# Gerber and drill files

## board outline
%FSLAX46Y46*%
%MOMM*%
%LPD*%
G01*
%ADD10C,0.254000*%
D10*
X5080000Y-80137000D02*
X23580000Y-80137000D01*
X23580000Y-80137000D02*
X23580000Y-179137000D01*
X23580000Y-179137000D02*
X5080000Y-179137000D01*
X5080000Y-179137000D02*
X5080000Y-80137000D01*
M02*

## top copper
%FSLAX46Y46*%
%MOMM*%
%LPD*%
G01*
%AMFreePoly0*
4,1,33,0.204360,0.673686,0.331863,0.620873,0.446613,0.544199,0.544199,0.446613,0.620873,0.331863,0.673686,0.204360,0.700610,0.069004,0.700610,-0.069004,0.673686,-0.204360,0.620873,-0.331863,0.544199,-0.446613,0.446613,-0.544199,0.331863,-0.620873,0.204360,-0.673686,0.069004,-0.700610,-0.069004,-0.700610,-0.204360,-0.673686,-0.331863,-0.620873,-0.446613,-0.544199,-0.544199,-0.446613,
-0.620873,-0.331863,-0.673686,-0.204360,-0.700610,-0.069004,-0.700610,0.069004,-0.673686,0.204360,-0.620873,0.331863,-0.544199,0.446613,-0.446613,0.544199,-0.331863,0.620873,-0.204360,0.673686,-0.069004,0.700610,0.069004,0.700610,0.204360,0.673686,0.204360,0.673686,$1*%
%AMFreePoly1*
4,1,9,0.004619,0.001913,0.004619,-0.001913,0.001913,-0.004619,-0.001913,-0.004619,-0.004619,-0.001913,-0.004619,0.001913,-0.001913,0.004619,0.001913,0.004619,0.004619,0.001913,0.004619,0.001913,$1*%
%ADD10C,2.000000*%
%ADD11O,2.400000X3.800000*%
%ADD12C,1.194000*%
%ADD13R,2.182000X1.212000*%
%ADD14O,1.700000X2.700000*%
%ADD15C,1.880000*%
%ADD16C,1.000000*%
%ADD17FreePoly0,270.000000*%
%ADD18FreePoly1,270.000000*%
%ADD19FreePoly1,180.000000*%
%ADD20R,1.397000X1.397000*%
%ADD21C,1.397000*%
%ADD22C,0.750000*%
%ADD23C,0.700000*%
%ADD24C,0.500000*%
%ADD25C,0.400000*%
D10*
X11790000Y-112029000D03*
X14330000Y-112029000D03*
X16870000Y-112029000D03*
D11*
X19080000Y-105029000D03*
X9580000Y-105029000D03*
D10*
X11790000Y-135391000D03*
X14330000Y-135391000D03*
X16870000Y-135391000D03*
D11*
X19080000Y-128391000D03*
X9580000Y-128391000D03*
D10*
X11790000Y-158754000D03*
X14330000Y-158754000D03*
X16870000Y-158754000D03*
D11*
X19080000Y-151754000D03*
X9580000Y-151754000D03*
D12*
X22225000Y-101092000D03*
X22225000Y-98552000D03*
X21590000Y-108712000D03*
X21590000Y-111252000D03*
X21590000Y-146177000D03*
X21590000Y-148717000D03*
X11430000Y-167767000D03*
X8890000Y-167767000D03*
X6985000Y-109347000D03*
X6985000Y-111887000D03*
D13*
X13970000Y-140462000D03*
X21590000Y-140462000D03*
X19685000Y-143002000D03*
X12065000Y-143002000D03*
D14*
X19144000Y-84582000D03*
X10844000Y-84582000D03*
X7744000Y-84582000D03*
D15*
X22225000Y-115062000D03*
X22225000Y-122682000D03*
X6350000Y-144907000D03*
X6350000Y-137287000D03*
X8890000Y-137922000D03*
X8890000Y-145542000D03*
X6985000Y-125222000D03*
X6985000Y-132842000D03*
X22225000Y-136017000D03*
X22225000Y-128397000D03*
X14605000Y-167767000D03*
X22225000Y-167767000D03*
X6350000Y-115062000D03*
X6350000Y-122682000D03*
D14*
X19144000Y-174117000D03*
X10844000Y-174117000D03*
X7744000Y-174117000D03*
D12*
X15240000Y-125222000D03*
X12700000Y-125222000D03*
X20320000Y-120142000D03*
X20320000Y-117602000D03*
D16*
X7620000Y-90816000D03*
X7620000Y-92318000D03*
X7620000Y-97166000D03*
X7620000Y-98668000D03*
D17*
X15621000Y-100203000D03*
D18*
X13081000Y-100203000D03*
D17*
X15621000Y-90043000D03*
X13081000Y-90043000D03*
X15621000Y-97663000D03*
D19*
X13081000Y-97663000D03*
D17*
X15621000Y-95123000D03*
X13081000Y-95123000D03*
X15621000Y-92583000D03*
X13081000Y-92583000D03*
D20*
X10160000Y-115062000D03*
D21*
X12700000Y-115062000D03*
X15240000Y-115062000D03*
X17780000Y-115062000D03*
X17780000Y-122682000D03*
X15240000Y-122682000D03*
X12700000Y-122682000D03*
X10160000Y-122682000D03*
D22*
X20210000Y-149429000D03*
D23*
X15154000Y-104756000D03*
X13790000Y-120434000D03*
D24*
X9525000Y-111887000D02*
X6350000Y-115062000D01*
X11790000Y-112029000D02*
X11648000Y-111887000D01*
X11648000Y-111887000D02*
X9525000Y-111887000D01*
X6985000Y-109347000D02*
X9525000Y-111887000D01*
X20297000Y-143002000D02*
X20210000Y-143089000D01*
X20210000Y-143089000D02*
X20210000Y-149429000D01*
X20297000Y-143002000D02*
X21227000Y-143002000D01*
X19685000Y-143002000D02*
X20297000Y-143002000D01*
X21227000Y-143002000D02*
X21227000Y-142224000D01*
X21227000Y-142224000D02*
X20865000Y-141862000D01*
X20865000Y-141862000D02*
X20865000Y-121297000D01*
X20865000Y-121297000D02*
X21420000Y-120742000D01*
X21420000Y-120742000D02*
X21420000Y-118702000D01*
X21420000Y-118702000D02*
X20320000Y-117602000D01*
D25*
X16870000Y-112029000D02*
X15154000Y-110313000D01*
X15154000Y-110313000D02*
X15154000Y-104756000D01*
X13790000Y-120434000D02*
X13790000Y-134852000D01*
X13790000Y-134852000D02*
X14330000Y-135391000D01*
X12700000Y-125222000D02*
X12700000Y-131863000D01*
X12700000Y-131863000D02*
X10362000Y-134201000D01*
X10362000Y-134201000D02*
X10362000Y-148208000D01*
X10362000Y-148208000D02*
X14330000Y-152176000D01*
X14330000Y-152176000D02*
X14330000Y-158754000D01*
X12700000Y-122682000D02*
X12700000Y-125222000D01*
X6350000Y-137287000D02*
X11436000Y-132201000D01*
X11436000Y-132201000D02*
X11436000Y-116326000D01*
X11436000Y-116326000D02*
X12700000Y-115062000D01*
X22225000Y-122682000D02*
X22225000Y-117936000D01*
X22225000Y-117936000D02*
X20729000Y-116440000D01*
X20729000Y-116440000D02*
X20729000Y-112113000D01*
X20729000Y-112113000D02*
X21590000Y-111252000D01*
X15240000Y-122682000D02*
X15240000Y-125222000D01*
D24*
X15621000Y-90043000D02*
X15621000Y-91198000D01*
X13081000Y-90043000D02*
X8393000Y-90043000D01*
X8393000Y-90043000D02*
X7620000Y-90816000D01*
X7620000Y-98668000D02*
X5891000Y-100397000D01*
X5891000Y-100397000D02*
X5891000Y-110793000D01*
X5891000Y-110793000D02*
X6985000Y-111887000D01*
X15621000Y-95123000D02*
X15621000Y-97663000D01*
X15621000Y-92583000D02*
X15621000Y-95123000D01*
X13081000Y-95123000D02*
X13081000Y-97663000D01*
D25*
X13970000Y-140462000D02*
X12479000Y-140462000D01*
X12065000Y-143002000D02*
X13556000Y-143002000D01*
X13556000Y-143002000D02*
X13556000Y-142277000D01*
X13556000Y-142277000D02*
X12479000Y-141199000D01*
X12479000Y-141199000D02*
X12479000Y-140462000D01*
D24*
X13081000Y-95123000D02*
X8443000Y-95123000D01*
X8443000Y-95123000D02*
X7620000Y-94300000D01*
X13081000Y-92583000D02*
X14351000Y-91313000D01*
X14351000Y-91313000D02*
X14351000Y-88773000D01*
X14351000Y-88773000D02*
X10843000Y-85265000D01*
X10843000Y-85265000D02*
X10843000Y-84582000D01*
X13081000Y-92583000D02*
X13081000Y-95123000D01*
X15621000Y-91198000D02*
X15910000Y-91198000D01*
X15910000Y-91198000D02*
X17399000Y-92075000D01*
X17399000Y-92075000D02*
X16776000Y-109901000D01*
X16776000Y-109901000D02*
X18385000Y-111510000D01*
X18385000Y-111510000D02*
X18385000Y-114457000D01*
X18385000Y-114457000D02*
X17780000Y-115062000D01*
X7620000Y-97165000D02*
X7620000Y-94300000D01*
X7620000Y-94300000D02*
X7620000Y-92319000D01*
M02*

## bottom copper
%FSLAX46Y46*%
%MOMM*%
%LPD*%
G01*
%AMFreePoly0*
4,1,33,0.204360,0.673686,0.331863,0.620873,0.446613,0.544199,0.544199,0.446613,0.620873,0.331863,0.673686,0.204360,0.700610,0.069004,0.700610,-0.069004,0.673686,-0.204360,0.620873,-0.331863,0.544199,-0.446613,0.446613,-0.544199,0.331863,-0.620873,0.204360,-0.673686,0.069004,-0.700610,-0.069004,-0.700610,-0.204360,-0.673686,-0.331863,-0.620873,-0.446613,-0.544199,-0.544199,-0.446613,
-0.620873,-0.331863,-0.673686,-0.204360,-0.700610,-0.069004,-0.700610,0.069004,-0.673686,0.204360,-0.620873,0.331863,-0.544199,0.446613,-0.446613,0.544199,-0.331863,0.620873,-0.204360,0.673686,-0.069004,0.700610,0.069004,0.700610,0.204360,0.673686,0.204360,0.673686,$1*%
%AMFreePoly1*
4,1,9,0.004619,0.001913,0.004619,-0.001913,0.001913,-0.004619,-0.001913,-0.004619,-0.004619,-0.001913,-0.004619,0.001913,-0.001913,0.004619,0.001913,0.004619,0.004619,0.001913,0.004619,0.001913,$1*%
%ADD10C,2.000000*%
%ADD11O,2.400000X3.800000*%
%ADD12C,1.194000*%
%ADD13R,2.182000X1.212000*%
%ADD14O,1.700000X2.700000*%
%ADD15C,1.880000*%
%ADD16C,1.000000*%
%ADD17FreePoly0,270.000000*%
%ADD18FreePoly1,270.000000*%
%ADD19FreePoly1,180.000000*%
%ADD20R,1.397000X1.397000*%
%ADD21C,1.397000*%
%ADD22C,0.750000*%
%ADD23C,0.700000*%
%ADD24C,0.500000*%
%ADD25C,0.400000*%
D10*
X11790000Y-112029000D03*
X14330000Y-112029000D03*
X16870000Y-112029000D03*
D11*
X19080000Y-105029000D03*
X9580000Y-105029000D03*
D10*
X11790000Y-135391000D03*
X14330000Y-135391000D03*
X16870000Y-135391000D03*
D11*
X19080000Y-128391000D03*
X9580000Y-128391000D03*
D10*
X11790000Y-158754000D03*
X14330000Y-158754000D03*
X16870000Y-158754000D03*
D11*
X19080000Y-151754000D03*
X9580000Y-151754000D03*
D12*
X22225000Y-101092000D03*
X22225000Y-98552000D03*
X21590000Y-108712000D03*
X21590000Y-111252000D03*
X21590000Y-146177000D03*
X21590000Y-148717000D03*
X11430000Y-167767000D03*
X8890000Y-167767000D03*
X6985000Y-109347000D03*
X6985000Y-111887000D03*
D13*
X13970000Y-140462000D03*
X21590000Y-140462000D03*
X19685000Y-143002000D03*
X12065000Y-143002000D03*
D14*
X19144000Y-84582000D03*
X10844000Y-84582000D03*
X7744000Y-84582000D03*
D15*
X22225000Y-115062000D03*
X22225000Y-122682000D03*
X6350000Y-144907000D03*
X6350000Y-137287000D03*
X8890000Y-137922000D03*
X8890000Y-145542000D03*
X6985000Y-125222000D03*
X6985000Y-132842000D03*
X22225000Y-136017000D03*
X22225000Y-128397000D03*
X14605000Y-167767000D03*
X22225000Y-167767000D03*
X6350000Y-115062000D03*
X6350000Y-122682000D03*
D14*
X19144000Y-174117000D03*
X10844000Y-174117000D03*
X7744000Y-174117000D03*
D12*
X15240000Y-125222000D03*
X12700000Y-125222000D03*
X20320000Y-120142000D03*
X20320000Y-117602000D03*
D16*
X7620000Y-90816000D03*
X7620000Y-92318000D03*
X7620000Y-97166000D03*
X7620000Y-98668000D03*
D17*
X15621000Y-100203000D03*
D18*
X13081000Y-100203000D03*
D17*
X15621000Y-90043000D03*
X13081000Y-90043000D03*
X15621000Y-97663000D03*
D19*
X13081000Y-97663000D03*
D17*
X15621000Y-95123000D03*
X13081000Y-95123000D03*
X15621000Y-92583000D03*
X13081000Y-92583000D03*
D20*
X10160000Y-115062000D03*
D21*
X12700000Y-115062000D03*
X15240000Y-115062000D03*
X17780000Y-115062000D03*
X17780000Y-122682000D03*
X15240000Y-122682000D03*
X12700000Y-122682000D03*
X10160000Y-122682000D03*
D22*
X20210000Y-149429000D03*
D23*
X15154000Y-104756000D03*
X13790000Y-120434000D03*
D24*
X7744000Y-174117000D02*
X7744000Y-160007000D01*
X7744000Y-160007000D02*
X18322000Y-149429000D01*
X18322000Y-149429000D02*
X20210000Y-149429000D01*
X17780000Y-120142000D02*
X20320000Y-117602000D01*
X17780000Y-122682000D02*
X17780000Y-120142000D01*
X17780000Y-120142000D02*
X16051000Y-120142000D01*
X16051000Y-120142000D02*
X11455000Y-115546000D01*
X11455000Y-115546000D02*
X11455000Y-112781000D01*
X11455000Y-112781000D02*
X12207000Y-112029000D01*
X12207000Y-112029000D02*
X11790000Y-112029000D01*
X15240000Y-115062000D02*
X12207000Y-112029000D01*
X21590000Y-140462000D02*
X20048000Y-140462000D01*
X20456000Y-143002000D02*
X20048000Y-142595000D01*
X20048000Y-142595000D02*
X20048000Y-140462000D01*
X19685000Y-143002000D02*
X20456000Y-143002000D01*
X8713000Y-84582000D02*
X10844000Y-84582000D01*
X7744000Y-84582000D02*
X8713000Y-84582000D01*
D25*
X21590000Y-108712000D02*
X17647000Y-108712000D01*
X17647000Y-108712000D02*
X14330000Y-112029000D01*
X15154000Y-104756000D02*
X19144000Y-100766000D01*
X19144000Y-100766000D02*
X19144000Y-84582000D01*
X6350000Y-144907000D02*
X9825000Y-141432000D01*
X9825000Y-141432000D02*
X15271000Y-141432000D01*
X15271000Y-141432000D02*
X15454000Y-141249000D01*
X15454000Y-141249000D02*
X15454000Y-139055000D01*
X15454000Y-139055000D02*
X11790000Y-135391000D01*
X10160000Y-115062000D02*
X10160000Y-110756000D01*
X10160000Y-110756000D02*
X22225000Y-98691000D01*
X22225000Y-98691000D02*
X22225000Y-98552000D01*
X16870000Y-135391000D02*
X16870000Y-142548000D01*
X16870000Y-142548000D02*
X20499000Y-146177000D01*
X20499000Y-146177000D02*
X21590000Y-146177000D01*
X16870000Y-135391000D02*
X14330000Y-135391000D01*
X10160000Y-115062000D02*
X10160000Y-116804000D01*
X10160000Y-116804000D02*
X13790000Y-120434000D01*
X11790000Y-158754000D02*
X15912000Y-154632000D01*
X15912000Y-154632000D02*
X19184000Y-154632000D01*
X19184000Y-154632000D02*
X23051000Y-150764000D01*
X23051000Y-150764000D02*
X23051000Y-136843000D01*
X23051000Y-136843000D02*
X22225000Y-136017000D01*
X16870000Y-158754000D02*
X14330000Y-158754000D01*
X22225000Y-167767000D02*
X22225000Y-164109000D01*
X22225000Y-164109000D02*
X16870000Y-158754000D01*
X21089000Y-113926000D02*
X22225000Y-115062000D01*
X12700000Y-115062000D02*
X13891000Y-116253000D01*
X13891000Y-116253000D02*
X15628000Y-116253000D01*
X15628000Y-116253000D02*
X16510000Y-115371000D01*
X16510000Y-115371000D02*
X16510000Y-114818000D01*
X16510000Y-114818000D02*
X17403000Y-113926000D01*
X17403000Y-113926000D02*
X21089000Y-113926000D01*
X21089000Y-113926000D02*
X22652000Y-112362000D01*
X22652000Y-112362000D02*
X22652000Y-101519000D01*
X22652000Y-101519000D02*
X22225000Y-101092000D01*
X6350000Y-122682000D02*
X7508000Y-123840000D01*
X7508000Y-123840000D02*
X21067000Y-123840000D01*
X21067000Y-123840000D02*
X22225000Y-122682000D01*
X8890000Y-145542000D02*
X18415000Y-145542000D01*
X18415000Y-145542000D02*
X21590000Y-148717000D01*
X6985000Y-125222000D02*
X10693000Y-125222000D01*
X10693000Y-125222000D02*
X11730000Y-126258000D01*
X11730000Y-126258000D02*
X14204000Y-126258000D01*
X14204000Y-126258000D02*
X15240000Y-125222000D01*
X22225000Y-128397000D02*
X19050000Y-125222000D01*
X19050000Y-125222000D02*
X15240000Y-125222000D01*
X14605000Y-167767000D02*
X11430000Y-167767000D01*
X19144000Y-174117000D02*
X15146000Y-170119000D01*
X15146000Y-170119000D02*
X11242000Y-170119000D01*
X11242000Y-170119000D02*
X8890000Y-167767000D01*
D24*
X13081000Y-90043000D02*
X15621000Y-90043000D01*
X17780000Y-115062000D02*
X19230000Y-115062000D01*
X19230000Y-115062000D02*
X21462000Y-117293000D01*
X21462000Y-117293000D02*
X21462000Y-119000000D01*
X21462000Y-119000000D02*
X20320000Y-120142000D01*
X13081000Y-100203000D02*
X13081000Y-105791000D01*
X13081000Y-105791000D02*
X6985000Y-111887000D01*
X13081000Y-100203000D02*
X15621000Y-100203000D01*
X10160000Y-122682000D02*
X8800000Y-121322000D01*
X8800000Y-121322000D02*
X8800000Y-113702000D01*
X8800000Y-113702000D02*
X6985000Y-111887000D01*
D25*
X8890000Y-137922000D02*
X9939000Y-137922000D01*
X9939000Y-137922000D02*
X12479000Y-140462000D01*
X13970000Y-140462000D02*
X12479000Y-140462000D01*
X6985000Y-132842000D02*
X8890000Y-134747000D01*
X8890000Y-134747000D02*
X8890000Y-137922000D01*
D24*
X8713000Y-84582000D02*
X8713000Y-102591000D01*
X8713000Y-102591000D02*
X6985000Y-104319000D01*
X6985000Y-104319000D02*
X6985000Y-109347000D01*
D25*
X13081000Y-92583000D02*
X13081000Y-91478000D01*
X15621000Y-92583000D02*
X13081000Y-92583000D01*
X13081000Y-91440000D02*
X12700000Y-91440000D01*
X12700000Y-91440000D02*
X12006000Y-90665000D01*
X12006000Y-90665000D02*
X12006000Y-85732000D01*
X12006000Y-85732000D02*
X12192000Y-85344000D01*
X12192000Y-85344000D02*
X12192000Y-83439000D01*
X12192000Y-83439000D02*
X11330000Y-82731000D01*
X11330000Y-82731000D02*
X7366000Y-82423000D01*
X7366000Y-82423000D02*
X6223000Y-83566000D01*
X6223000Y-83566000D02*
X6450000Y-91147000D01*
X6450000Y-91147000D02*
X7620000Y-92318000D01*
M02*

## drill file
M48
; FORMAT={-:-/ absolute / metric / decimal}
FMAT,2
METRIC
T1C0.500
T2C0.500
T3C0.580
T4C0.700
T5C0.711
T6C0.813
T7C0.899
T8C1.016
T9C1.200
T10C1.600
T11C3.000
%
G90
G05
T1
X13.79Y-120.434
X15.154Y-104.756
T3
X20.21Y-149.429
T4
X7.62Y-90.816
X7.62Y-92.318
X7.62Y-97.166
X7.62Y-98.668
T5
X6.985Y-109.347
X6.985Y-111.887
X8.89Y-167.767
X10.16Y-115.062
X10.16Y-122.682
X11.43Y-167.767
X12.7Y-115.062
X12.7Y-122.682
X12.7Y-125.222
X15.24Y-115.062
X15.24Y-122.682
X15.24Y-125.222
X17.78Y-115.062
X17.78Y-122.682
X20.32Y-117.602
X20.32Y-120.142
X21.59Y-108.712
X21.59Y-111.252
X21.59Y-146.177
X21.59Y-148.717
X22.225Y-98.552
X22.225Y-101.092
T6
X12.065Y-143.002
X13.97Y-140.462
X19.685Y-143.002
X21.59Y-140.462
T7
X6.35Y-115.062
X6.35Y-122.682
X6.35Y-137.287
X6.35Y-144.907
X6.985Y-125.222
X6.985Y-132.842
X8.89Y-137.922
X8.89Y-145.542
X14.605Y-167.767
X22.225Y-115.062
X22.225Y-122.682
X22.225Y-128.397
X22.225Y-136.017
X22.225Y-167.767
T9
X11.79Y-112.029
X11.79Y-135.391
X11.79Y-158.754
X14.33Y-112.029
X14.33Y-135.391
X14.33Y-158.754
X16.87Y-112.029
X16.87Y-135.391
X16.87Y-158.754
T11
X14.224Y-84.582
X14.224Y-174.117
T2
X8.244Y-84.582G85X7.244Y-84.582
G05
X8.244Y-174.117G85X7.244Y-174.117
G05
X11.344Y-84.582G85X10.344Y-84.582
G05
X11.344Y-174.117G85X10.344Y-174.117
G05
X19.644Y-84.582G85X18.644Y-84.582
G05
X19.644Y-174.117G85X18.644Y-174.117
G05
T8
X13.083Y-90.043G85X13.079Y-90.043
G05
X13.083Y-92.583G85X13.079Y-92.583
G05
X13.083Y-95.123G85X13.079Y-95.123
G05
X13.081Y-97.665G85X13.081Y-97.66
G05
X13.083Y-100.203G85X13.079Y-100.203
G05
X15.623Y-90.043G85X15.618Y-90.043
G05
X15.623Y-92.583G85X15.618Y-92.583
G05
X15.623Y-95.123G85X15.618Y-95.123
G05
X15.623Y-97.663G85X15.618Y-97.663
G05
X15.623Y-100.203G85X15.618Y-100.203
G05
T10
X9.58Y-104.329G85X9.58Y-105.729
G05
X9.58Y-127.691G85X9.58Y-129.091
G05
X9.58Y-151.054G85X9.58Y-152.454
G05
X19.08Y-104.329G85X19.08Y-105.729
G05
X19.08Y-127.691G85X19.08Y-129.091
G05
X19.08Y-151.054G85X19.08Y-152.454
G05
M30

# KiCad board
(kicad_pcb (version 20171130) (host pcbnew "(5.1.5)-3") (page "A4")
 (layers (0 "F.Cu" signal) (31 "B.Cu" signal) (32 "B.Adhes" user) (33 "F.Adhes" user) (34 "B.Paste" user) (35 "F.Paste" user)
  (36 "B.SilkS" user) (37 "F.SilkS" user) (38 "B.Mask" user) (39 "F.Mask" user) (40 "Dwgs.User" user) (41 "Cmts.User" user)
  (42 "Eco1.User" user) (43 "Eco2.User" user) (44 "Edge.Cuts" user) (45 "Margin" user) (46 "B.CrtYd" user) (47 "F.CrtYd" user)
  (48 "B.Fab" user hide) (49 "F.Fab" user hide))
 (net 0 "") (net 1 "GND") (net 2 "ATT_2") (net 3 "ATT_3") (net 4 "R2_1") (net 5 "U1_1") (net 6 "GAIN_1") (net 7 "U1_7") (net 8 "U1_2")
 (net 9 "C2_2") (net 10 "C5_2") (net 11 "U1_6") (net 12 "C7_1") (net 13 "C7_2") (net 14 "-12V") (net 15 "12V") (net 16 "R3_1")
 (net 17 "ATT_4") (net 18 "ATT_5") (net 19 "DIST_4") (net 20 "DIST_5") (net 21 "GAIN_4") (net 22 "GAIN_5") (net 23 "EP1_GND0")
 (segment (start 7.744 174.117) (end 7.744 160.007) (width 0.5) (layer "B.Cu") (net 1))
 (segment (start 7.744 160.007) (end 18.322 149.429) (width 0.5) (layer "B.Cu") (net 1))
 (segment (start 18.322 149.429) (end 20.21 149.429) (width 0.5) (layer "B.Cu") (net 1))
 (segment (start 17.78 120.142) (end 20.32 117.602) (width 0.5) (layer "B.Cu") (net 1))
 (segment (start 17.78 122.682) (end 17.78 120.142) (width 0.5) (layer "B.Cu") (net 1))
 (segment (start 17.78 120.142) (end 16.051 120.142) (width 0.5) (layer "B.Cu") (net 1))
 (segment (start 16.051 120.142) (end 11.455 115.546) (width 0.5) (layer "B.Cu") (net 1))
 (segment (start 11.455 115.546) (end 11.455 112.781) (width 0.5) (layer "B.Cu") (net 1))
 (segment (start 11.455 112.781) (end 12.207 112.029) (width 0.5) (layer "B.Cu") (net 1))
 (segment (start 12.207 112.029) (end 11.79 112.029) (width 0.5) (layer "B.Cu") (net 1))
 (segment (start 15.24 115.062) (end 12.207 112.029) (width 0.5) (layer "B.Cu") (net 1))
 (segment (start 21.59 140.462) (end 20.048 140.462) (width 0.5) (layer "B.Cu") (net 1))
 (segment (start 20.456 143.002) (end 20.048 142.595) (width 0.5) (layer "B.Cu") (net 1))
 (segment (start 20.048 142.595) (end 20.048 140.462) (width 0.5) (layer "B.Cu") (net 1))
 (segment (start 19.685 143.002) (end 20.456 143.002) (width 0.5) (layer "B.Cu") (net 1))
 (segment (start 8.713 84.582) (end 10.844 84.582) (width 0.5) (layer "B.Cu") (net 1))
 (segment (start 7.744 84.582) (end 8.713 84.582) (width 0.5) (layer "B.Cu") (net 1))
 (segment (start 21.59 108.712) (end 17.647 108.712) (width 0.4) (layer "B.Cu") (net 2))
 (segment (start 17.647 108.712) (end 14.33 112.029) (width 0.4) (layer "B.Cu") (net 2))
 (segment (start 15.154 104.756) (end 19.144 100.766) (width 0.4) (layer "B.Cu") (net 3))
 (segment (start 19.144 100.766) (end 19.144 84.582) (width 0.4) (layer "B.Cu") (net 3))
 (segment (start 6.35 144.907) (end 9.825 141.432) (width 0.4) (layer "B.Cu") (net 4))
 (segment (start 9.825 141.432) (end 15.271 141.432) (width 0.4) (layer "B.Cu") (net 4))
 (segment (start 15.271 141.432) (end 15.454 141.249) (width 0.4) (layer "B.Cu") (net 4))
 (segment (start 15.454 141.249) (end 15.454 139.055) (width 0.4) (layer "B.Cu") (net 4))
 (segment (start 15.454 139.055) (end 11.79 135.391) (width 0.4) (layer "B.Cu") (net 4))
 (segment (start 10.16 115.062) (end 10.16 110.756) (width 0.4) (layer "B.Cu") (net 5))
 (segment (start 10.16 110.756) (end 22.225 98.691) (width 0.4) (layer "B.Cu") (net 5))
 (segment (start 22.225 98.691) (end 22.225 98.552) (width 0.4) (layer "B.Cu") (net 5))
 (segment (start 16.87 135.391) (end 16.87 142.548) (width 0.4) (layer "B.Cu") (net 5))
 (segment (start 16.87 142.548) (end 20.499 146.177) (width 0.4) (layer "B.Cu") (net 5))
 (segment (start 20.499 146.177) (end 21.59 146.177) (width 0.4) (layer "B.Cu") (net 5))
 (segment (start 16.87 135.391) (end 14.33 135.391) (width 0.4) (layer "B.Cu") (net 5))
 (segment (start 10.16 115.062) (end 10.16 116.804) (width 0.4) (layer "B.Cu") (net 5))
 (segment (start 10.16 116.804) (end 13.79 120.434) (width 0.4) (layer "B.Cu") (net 5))
 (segment (start 11.79 158.754) (end 15.912 154.632) (width 0.4) (layer "B.Cu") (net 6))
 (segment (start 15.912 154.632) (end 19.184 154.632) (width 0.4) (layer "B.Cu") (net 6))
 (segment (start 19.184 154.632) (end 23.051 150.764) (width 0.4) (layer "B.Cu") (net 6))
 (segment (start 23.051 150.764) (end 23.051 136.843) (width 0.4) (layer "B.Cu") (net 6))
 (segment (start 23.051 136.843) (end 22.225 136.017) (width 0.4) (layer "B.Cu") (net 6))
 (segment (start 16.87 158.754) (end 14.33 158.754) (width 0.4) (layer "B.Cu") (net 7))
 (segment (start 22.225 167.767) (end 22.225 164.109) (width 0.4) (layer "B.Cu") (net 7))
 (segment (start 22.225 164.109) (end 16.87 158.754) (width 0.4) (layer "B.Cu") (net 7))
 (segment (start 21.089 113.926) (end 22.225 115.062) (width 0.4) (layer "B.Cu") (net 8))
 (segment (start 12.7 115.062) (end 13.891 116.253) (width 0.4) (layer "B.Cu") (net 8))
 (segment (start 13.891 116.253) (end 15.628 116.253) (width 0.4) (layer "B.Cu") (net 8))
 (segment (start 15.628 116.253) (end 16.51 115.371) (width 0.4) (layer "B.Cu") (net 8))
 (segment (start 16.51 115.371) (end 16.51 114.818) (width 0.4) (layer "B.Cu") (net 8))
 (segment (start 16.51 114.818) (end 17.403 113.926) (width 0.4) (layer "B.Cu") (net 8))
 (segment (start 17.403 113.926) (end 21.089 113.926) (width 0.4) (layer "B.Cu") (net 8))
 (segment (start 21.089 113.926) (end 22.652 112.362) (width 0.4) (layer "B.Cu") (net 8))
 (segment (start 22.652 112.362) (end 22.652 101.519) (width 0.4) (layer "B.Cu") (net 8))
 (segment (start 22.652 101.519) (end 22.225 101.092) (width 0.4) (layer "B.Cu") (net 8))
 (segment (start 6.35 122.682) (end 7.508 123.84) (width 0.4) (layer "B.Cu") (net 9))
 (segment (start 7.508 123.84) (end 21.067 123.84) (width 0.4) (layer "B.Cu") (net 9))
 (segment (start 21.067 123.84) (end 22.225 122.682) (width 0.4) (layer "B.Cu") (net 9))
 (segment (start 8.89 145.542) (end 18.415 145.542) (width 0.4) (layer "B.Cu") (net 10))
 (segment (start 18.415 145.542) (end 21.59 148.717) (width 0.4) (layer "B.Cu") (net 10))
 (segment (start 6.985 125.222) (end 10.693 125.222) (width 0.4) (layer "B.Cu") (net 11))
 (segment (start 10.693 125.222) (end 11.73 126.258) (width 0.4) (layer "B.Cu") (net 11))
 (segment (start 11.73 126.258) (end 14.204 126.258) (width 0.4) (layer "B.Cu") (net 11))
 (segment (start 14.204 126.258) (end 15.24 125.222) (width 0.4) (layer "B.Cu") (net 11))
 (segment (start 22.225 128.397) (end 19.05 125.222) (width 0.4) (layer "B.Cu") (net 11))
 (segment (start 19.05 125.222) (end 15.24 125.222) (width 0.4) (layer "B.Cu") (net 11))
 (segment (start 14.605 167.767) (end 11.43 167.767) (width 0.4) (layer "B.Cu") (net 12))
 (segment (start 19.144 174.117) (end 15.146 170.119) (width 0.4) (layer "B.Cu") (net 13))
 (segment (start 15.146 170.119) (end 11.242 170.119) (width 0.4) (layer "B.Cu") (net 13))
 (segment (start 11.242 170.119) (end 8.89 167.767) (width 0.4) (layer "B.Cu") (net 13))
 (segment (start 13.081 90.043) (end 15.621 90.043) (width 0.5) (layer "B.Cu") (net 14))
 (segment (start 17.78 115.062) (end 19.23 115.062) (width 0.5) (layer "B.Cu") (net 14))
 (segment (start 19.23 115.062) (end 21.462 117.293) (width 0.5) (layer "B.Cu") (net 14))
 (segment (start 21.462 117.293) (end 21.462 119) (width 0.5) (layer "B.Cu") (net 14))
 (segment (start 21.462 119) (end 20.32 120.142) (width 0.5) (layer "B.Cu") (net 14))
 (segment (start 13.081 100.203) (end 13.081 105.791) (width 0.5) (layer "B.Cu") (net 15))
 (segment (start 13.081 105.791) (end 6.985 111.887) (width 0.5) (layer "B.Cu") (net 15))
 (segment (start 13.081 100.203) (end 15.621 100.203) (width 0.5) (layer "B.Cu") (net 15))
 (segment (start 10.16 122.682) (end 8.8 121.322) (width 0.5) (layer "B.Cu") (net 15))
 (segment (start 8.8 121.322) (end 8.8 113.702) (width 0.5) (layer "B.Cu") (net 15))
 (segment (start 8.8 113.702) (end 6.985 111.887) (width 0.5) (layer "B.Cu") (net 15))
 (segment (start 8.89 137.922) (end 9.939 137.922) (width 0.4) (layer "B.Cu") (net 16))
 (segment (start 9.939 137.922) (end 12.479 140.462) (width 0.4) (layer "B.Cu") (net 16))
 (segment (start 13.97 140.462) (end 12.479 140.462) (width 0.4) (layer "B.Cu") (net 16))
 (segment (start 6.985 132.842) (end 8.89 134.747) (width 0.4) (layer "B.Cu") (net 16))
 (segment (start 8.89 134.747) (end 8.89 137.922) (width 0.4) (layer "B.Cu") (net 16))
 (segment (start 8.713 84.582) (end 8.713 102.591) (width 0.5) (layer "B.Cu") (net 1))
 (segment (start 8.713 102.591) (end 6.985 104.319) (width 0.5) (layer "B.Cu") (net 1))
 (segment (start 6.985 104.319) (end 6.985 109.347) (width 0.5) (layer "B.Cu") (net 1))
 (segment (start 13.081 92.583) (end 13.081 91.478) (width 0.4) (layer "B.Cu") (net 1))
 (segment (start 15.621 92.583) (end 13.081 92.583) (width 0.4) (layer "B.Cu") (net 1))
 (segment (start 13.081 91.44) (end 12.7 91.44) (width 0.4) (layer "B.Cu") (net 1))
 (segment (start 12.7 91.44) (end 12.006 90.665) (width 0.4) (layer "B.Cu") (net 1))
 (segment (start 12.006 90.665) (end 12.006 85.732) (width 0.4) (layer "B.Cu") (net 1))
 (segment (start 12.006 85.732) (end 12.192 85.344) (width 0.4) (layer "B.Cu") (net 1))
 (segment (start 12.192 85.344) (end 12.192 83.439) (width 0.4) (layer "B.Cu") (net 1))
 (segment (start 12.192 83.439) (end 11.33 82.731) (width 0.4) (layer "B.Cu") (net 1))
 (segment (start 11.33 82.731) (end 7.366 82.423) (width 0.4) (layer "B.Cu") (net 1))
 (segment (start 7.366 82.423) (end 6.223 83.566) (width 0.4) (layer "B.Cu") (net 1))
 (segment (start 6.223 83.566) (end 6.45 91.147) (width 0.4) (layer "B.Cu") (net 1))
 (segment (start 6.45 91.147) (end 7.62 92.318) (width 0.4) (layer "B.Cu") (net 1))
 (gr_line (start 5.08 80.137) (end 23.58 80.137) (width 0.254) (layer "Edge.Cuts"))
 (gr_line (start 23.58 80.137) (end 23.58 179.137) (width 0.254) (layer "Edge.Cuts"))
 (gr_line (start 23.58 179.137) (end 5.08 179.137) (width 0.254) (layer "Edge.Cuts"))
 (gr_line (start 5.08 179.137) (end 5.08 80.137) (width 0.254) (layer "Edge.Cuts"))
 (segment (start 9.525 111.887) (end 6.35 115.062) (width 0.5) (layer "F.Cu") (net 1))
 (segment (start 11.79 112.029) (end 11.648 111.887) (width 0.5) (layer "F.Cu") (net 1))
 (segment (start 11.648 111.887) (end 9.525 111.887) (width 0.5) (layer "F.Cu") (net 1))
 (segment (start 6.985 109.347) (end 9.525 111.887) (width 0.5) (layer "F.Cu") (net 1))
 (segment (start 20.297 143.002) (end 20.21 143.089) (width 0.5) (layer "F.Cu") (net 1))
 (segment (start 20.21 143.089) (end 20.21 149.429) (width 0.5) (layer "F.Cu") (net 1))
 (segment (start 20.297 143.002) (end 21.227 143.002) (width 0.5) (layer "F.Cu") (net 1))
 (segment (start 19.685 143.002) (end 20.297 143.002) (width 0.5) (layer "F.Cu") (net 1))
 (segment (start 21.227 143.002) (end 21.227 142.224) (width 0.5) (layer "F.Cu") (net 1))
 (segment (start 21.227 142.224) (end 20.865 141.862) (width 0.5) (layer "F.Cu") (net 1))
 (segment (start 20.865 141.862) (end 20.865 121.297) (width 0.5) (layer "F.Cu") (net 1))
 (segment (start 20.865 121.297) (end 21.42 120.742) (width 0.5) (layer "F.Cu") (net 1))
 (segment (start 21.42 120.742) (end 21.42 118.702) (width 0.5) (layer "F.Cu") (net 1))
 (segment (start 21.42 118.702) (end 20.32 117.602) (width 0.5) (layer "F.Cu") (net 1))
 (segment (start 16.87 112.029) (end 15.154 110.313) (width 0.4) (layer "F.Cu") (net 3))
 (segment (start 15.154 110.313) (end 15.154 104.756) (width 0.4) (layer "F.Cu") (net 3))
 (segment (start 13.79 120.434) (end 13.79 134.852) (width 0.4) (layer "F.Cu") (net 5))
 (segment (start 13.79 134.852) (end 14.33 135.391) (width 0.4) (layer "F.Cu") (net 5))
 (segment (start 12.7 125.222) (end 12.7 131.863) (width 0.4) (layer "F.Cu") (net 7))
 (segment (start 12.7 131.863) (end 10.362 134.201) (width 0.4) (layer "F.Cu") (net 7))
 (segment (start 10.362 134.201) (end 10.362 148.208) (width 0.4) (layer "F.Cu") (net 7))
 (segment (start 10.362 148.208) (end 14.33 152.176) (width 0.4) (layer "F.Cu") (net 7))
 (segment (start 14.33 152.176) (end 14.33 158.754) (width 0.4) (layer "F.Cu") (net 7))
 (segment (start 12.7 122.682) (end 12.7 125.222) (width 0.4) (layer "F.Cu") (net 7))
 (segment (start 6.35 137.287) (end 11.436 132.201) (width 0.4) (layer "F.Cu") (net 8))
 (segment (start 11.436 132.201) (end 11.436 116.326) (width 0.4) (layer "F.Cu") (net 8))
 (segment (start 11.436 116.326) (end 12.7 115.062) (width 0.4) (layer "F.Cu") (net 8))
 (segment (start 22.225 122.682) (end 22.225 117.936) (width 0.4) (layer "F.Cu") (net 9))
 (segment (start 22.225 117.936) (end 20.729 116.44) (width 0.4) (layer "F.Cu") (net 9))
 (segment (start 20.729 116.44) (end 20.729 112.113) (width 0.4) (layer "F.Cu") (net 9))
 (segment (start 20.729 112.113) (end 21.59 111.252) (width 0.4) (layer "F.Cu") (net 9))
 (segment (start 15.24 122.682) (end 15.24 125.222) (width 0.4) (layer "F.Cu") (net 11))
 (segment (start 15.621 90.043) (end 15.621 91.198) (width 0.5) (layer "F.Cu") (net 14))
 (segment (start 13.081 90.043) (end 8.393 90.043) (width 0.5) (layer "F.Cu") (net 14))
 (segment (start 8.393 90.043) (end 7.62 90.816) (width 0.5) (layer "F.Cu") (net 14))
 (segment (start 7.62 98.668) (end 5.891 100.397) (width 0.5) (layer "F.Cu") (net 15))
 (segment (start 5.891 100.397) (end 5.891 110.793) (width 0.5) (layer "F.Cu") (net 15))
 (segment (start 5.891 110.793) (end 6.985 111.887) (width 0.5) (layer "F.Cu") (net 15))
 (segment (start 15.621 95.123) (end 15.621 97.663) (width 0.5) (layer "F.Cu") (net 1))
 (segment (start 15.621 92.583) (end 15.621 95.123) (width 0.5) (layer "F.Cu") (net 1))
 (segment (start 13.081 95.123) (end 13.081 97.663) (width 0.5) (layer "F.Cu") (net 1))
 (segment (start 13.97 140.462) (end 12.479 140.462) (width 0.4) (layer "F.Cu") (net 16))
 (segment (start 12.065 143.002) (end 13.556 143.002) (width 0.4) (layer "F.Cu") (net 16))
 (segment (start 13.556 143.002) (end 13.556 142.277) (width 0.4) (layer "F.Cu") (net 16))
 (segment (start 13.556 142.277) (end 12.479 141.199) (width 0.4) (layer "F.Cu") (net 16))
 (segment (start 12.479 141.199) (end 12.479 140.462) (width 0.4) (layer "F.Cu") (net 16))
 (segment (start 13.081 95.123) (end 8.443 95.123) (width 0.5) (layer "F.Cu") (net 1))
 (segment (start 8.443 95.123) (end 7.62 94.3) (width 0.5) (layer "F.Cu") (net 1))
 (segment (start 13.081 92.583) (end 14.351 91.313) (width 0.5) (layer "F.Cu") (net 1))
 (segment (start 14.351 91.313) (end 14.351 88.773) (width 0.5) (layer "F.Cu") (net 1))
 (segment (start 14.351 88.773) (end 10.843 85.265) (width 0.5) (layer "F.Cu") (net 1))
 (segment (start 10.843 85.265) (end 10.843 84.582) (width 0.5) (layer "F.Cu") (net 1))
 (segment (start 13.081 92.583) (end 13.081 95.123) (width 0.5) (layer "F.Cu") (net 1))
 (segment (start 15.621 91.198) (end 15.91 91.198) (width 0.5) (layer "F.Cu") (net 14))
 (segment (start 15.91 91.198) (end 17.399 92.075) (width 0.5) (layer "F.Cu") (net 14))
 (segment (start 17.399 92.075) (end 16.776 109.901) (width 0.5) (layer "F.Cu") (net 14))
 (segment (start 16.776 109.901) (end 18.385 111.51) (width 0.5) (layer "F.Cu") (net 14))
 (segment (start 18.385 111.51) (end 18.385 114.457) (width 0.5) (layer "F.Cu") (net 14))
 (segment (start 18.385 114.457) (end 17.78 115.062) (width 0.5) (layer "F.Cu") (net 14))
 (segment (start 7.62 97.165) (end 7.62 94.3) (width 0.5) (layer "F.Cu") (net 1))
 (segment (start 7.62 94.3) (end 7.62 92.319) (width 0.5) (layer "F.Cu") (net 1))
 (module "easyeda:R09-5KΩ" (layer "F.Cu") (at 14.33 108.529)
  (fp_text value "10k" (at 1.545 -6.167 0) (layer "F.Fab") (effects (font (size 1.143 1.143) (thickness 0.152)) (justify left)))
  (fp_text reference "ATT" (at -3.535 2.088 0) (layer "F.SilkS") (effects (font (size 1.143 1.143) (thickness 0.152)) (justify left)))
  (pad 1 thru_hole circle (at -2.54 3.5 0) (size 2 2) (layers "*.Cu" "*.Paste" "*.Mask") (drill 1.2) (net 1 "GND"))
  (pad 2 thru_hole circle (at 0 3.5 0) (size 2 2) (layers "*.Cu" "*.Paste" "*.Mask") (drill 1.2) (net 2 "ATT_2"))
  (pad 3 thru_hole circle (at 2.54 3.5 0) (size 2 2) (layers "*.Cu" "*.Paste" "*.Mask") (drill 1.2) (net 3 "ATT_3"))
  (pad 4 thru_hole oval (at 4.75 -3.5 0) (size 2.4 3.8) (layers "*.Cu" "*.Paste" "*.Mask") (drill oval 1.6 3) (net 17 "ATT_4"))
  (pad 5 thru_hole oval (at -4.75 -3.5 0) (size 2.4 3.8) (layers "*.Cu" "*.Paste" "*.Mask") (drill oval 1.6 3) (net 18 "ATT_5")))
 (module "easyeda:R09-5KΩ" (layer "F.Cu") (at 14.33 131.891)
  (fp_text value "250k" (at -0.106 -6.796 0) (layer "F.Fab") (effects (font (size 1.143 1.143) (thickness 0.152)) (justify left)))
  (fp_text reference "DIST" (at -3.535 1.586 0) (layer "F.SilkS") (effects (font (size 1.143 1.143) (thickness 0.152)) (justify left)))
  (pad 1 thru_hole circle (at -2.54 3.5 0) (size 2 2) (layers "*.Cu" "*.Paste" "*.Mask") (drill 1.2) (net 4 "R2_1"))
  (pad 2 thru_hole circle (at 0 3.5 0) (size 2 2) (layers "*.Cu" "*.Paste" "*.Mask") (drill 1.2) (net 5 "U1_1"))
  (pad 3 thru_hole circle (at 2.54 3.5 0) (size 2 2) (layers "*.Cu" "*.Paste" "*.Mask") (drill 1.2) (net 5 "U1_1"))
  (pad 4 thru_hole oval (at 4.75 -3.5 0) (size 2.4 3.8) (layers "*.Cu" "*.Paste" "*.Mask") (drill oval 1.6 3) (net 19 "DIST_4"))
  (pad 5 thru_hole oval (at -4.75 -3.5 0) (size 2.4 3.8) (layers "*.Cu" "*.Paste" "*.Mask") (drill oval 1.6 3) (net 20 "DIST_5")))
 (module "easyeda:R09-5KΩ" (layer "F.Cu") (at 14.33 155.254)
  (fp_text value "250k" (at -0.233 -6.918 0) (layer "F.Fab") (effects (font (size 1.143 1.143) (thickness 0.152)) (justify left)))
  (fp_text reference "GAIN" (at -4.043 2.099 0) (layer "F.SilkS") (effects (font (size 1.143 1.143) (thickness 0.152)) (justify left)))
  (pad 1 thru_hole circle (at -2.54 3.5 0) (size 2 2) (layers "*.Cu" "*.Paste" "*.Mask") (drill 1.2) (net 6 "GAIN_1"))
  (pad 2 thru_hole circle (at 0 3.5 0) (size 2 2) (layers "*.Cu" "*.Paste" "*.Mask") (drill 1.2) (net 7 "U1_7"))
  (pad 3 thru_hole circle (at 2.54 3.5 0) (size 2 2) (layers "*.Cu" "*.Paste" "*.Mask") (drill 1.2) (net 7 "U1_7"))
  (pad 4 thru_hole oval (at 4.75 -3.5 0) (size 2.4 3.8) (layers "*.Cu" "*.Paste" "*.Mask") (drill oval 1.6 3) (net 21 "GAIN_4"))
  (pad 5 thru_hole oval (at -4.75 -3.5 0) (size 2.4 3.8) (layers "*.Cu" "*.Paste" "*.Mask") (drill oval 1.6 3) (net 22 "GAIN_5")))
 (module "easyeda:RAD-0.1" (layer "F.Cu") (at 22.225 99.822 90)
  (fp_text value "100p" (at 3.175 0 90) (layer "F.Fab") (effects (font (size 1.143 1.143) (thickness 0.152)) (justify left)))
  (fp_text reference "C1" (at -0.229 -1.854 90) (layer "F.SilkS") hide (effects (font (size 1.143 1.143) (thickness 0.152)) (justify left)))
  (pad 1 thru_hole circle (at -1.27 0 90) (size 1.194 1.194) (layers "*.Cu" "*.Paste" "*.Mask") (drill 0.711) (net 8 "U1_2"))
  (pad 2 thru_hole circle (at 1.27 0 90) (size 1.194 1.194) (layers "*.Cu" "*.Paste" "*.Mask") (drill 0.711) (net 5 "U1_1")))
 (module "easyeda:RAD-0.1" (layer "F.Cu") (at 21.59 109.982 -90)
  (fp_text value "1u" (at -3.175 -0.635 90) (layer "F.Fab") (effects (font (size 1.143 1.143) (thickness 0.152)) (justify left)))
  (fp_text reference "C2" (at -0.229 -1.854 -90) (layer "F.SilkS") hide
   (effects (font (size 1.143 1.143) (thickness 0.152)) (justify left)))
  (pad 1 thru_hole circle (at -1.27 0 -90) (size 1.194 1.194) (layers "*.Cu" "*.Paste" "*.Mask") (drill 0.711) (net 2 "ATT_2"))
  (pad 2 thru_hole circle (at 1.27 0 -90) (size 1.194 1.194) (layers "*.Cu" "*.Paste" "*.Mask") (drill 0.711) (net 9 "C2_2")))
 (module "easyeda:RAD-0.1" (layer "F.Cu") (at 21.59 147.447 -90)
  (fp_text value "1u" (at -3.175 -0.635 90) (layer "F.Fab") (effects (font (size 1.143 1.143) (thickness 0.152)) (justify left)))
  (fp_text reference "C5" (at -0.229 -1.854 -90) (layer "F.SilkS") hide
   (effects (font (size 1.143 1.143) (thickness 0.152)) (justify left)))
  (pad 1 thru_hole circle (at -1.27 0 -90) (size 1.194 1.194) (layers "*.Cu" "*.Paste" "*.Mask") (drill 0.711) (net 5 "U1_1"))
  (pad 2 thru_hole circle (at 1.27 0 -90) (size 1.194 1.194) (layers "*.Cu" "*.Paste" "*.Mask") (drill 0.711) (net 10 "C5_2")))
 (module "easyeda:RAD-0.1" (layer "F.Cu") (at 10.16 167.767 180)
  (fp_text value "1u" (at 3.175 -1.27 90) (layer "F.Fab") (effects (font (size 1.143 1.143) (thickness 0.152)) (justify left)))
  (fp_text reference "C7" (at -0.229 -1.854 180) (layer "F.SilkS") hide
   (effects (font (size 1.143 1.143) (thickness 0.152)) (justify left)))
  (pad 1 thru_hole circle (at -1.27 0 180) (size 1.194 1.194) (layers "*.Cu" "*.Paste" "*.Mask") (drill 0.711) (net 12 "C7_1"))
  (pad 2 thru_hole circle (at 1.27 0 180) (size 1.194 1.194) (layers "*.Cu" "*.Paste" "*.Mask") (drill 0.711) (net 13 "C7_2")))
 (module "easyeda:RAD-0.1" (layer "F.Cu") (at 6.985 110.617 -90)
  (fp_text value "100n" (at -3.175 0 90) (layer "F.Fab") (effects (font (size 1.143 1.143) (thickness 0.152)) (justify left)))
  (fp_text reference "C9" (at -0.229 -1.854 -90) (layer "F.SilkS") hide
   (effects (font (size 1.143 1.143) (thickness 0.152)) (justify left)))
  (pad 1 thru_hole circle (at -1.27 0 -90) (size 1.194 1.194) (layers "*.Cu" "*.Paste" "*.Mask") (drill 0.711) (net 1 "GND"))
  (pad 2 thru_hole circle (at 1.27 0 -90) (size 1.194 1.194) (layers "*.Cu" "*.Paste" "*.Mask") (drill 0.711) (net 15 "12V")))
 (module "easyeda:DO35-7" (layer "F.Cu") (at 17.78 140.462)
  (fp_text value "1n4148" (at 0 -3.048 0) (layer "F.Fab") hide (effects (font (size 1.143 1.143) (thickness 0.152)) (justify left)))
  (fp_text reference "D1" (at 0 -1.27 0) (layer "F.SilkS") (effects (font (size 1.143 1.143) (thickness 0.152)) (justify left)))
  (pad "C" thru_hole rect (at -3.81 0 0) (size 2.182 1.212) (layers "*.Cu" "*.Paste" "*.Mask") (drill 0.813) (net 16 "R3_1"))
  (pad "A" thru_hole rect (at 3.81 0 0) (size 2.182 1.212) (layers "*.Cu" "*.Paste" "*.Mask") (drill 0.813) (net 1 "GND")))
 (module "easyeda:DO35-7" (layer "F.Cu") (at 15.875 143.002 180)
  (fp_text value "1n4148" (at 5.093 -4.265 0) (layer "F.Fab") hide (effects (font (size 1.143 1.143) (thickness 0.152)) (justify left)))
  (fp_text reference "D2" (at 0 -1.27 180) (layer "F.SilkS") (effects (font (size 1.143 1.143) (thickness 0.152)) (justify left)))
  (pad "C" thru_hole rect (at -3.81 0 180) (size 2.182 1.212) (layers "*.Cu" "*.Paste" "*.Mask") (drill 0.813) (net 1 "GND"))
  (pad "A" thru_hole rect (at 3.81 0 180) (size 2.182 1.212) (layers "*.Cu" "*.Paste" "*.Mask") (drill 0.813) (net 16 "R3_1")))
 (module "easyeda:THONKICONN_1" (layer "F.Cu") (at 14.224 84.582 -90)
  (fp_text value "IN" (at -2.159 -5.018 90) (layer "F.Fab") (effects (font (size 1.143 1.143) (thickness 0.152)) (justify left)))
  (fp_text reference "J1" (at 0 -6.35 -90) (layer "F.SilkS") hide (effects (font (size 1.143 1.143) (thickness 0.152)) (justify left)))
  (pad "" np_thru_hole circle (at 0 0) (size 3 3) (drill 3) (layers "*.Cu" "*.Mask"))
  (pad 3 thru_hole oval (at 0 -4.92 -90) (size 2.7 1.7) (layers "*.Cu" "*.Paste" "*.Mask") (drill oval 0.5 1.5) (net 3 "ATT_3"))
  (pad 2 thru_hole oval (at 0 3.38 -90) (size 2.7 1.7) (layers "*.Cu" "*.Paste" "*.Mask") (drill oval 0.5 1.5) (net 1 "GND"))
  (pad 1 thru_hole oval (at 0 6.48 -90) (size 2.7 1.7) (layers "*.Cu" "*.Paste" "*.Mask") (drill oval 0.5 1.5) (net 1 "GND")))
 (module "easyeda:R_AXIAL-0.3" (layer "F.Cu") (at 22.225 118.872 -90)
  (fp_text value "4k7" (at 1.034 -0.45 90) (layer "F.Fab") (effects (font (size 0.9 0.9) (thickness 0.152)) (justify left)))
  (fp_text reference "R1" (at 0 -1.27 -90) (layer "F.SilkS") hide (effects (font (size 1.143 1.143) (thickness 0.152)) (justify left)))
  (pad 1 thru_hole circle (at -3.81 0 -90) (size 1.88 1.88) (layers "*.Cu" "*.Paste" "*.Mask") (drill 0.899) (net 8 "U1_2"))
  (pad 2 thru_hole circle (at 3.81 0 -90) (size 1.88 1.88) (layers "*.Cu" "*.Paste" "*.Mask") (drill 0.899) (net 9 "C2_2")))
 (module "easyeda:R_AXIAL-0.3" (layer "F.Cu") (at 6.35 141.097 90)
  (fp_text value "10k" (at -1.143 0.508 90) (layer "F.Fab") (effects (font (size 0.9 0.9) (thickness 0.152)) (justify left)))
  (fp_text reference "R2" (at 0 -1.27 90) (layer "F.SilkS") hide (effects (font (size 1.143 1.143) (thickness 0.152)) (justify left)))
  (pad 1 thru_hole circle (at -3.81 0 90) (size 1.88 1.88) (layers "*.Cu" "*.Paste" "*.Mask") (drill 0.899) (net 4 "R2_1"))
  (pad 2 thru_hole circle (at 3.81 0 90) (size 1.88 1.88) (layers "*.Cu" "*.Paste" "*.Mask") (drill 0.899) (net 8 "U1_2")))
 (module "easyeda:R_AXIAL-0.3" (layer "F.Cu") (at 8.89 141.732 -90)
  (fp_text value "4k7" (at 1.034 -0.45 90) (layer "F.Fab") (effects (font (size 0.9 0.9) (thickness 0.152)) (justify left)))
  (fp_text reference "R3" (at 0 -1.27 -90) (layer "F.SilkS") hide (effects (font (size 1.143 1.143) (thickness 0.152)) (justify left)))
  (pad 1 thru_hole circle (at -3.81 0 -90) (size 1.88 1.88) (layers "*.Cu" "*.Paste" "*.Mask") (drill 0.899) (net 16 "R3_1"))
  (pad 2 thru_hole circle (at 3.81 0 -90) (size 1.88 1.88) (layers "*.Cu" "*.Paste" "*.Mask") (drill 0.899) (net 10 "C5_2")))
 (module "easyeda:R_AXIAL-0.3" (layer "F.Cu") (at 6.985 129.032 -90)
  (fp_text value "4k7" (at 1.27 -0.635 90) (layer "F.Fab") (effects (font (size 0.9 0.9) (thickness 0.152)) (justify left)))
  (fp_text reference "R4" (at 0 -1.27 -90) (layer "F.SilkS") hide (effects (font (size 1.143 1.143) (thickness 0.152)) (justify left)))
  (pad 1 thru_hole circle (at -3.81 0 -90) (size 1.88 1.88) (layers "*.Cu" "*.Paste" "*.Mask") (drill 0.899) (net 11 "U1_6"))
  (pad 2 thru_hole circle (at 3.81 0 -90) (size 1.88 1.88) (layers "*.Cu" "*.Paste" "*.Mask") (drill 0.899) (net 16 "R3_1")))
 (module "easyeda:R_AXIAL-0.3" (layer "F.Cu") (at 22.225 132.207 90)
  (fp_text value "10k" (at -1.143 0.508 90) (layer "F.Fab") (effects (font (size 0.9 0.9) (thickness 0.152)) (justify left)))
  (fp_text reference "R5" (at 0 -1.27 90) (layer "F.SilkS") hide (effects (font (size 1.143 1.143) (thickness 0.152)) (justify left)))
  (pad 1 thru_hole circle (at -3.81 0 90) (size 1.88 1.88) (layers "*.Cu" "*.Paste" "*.Mask") (drill 0.899) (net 6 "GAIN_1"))
  (pad 2 thru_hole circle (at 3.81 0 90) (size 1.88 1.88) (layers "*.Cu" "*.Paste" "*.Mask") (drill 0.899) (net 11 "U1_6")))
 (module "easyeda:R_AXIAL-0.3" (layer "F.Cu") (at 18.415 167.767)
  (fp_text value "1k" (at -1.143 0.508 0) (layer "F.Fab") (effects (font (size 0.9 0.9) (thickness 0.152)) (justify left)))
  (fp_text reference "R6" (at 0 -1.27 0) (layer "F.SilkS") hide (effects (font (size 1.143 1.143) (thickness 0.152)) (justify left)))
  (pad 1 thru_hole circle (at -3.81 0 0) (size 1.88 1.88) (layers "*.Cu" "*.Paste" "*.Mask") (drill 0.899) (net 12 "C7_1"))
  (pad 2 thru_hole circle (at 3.81 0 0) (size 1.88 1.88) (layers "*.Cu" "*.Paste" "*.Mask") (drill 0.899) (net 7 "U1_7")))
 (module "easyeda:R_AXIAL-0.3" (layer "F.Cu") (at 6.35 118.872 -90)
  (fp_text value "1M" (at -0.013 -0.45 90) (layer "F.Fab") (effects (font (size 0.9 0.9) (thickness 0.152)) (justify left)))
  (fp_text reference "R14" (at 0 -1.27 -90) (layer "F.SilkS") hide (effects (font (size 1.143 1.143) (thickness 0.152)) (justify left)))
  (pad 1 thru_hole circle (at -3.81 0 -90) (size 1.88 1.88) (layers "*.Cu" "*.Paste" "*.Mask") (drill 0.899) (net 1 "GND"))
  (pad 2 thru_hole circle (at 3.81 0 -90) (size 1.88 1.88) (layers "*.Cu" "*.Paste" "*.Mask") (drill 0.899) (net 9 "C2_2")))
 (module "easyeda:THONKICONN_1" (layer "F.Cu") (at 14.224 174.117 -90)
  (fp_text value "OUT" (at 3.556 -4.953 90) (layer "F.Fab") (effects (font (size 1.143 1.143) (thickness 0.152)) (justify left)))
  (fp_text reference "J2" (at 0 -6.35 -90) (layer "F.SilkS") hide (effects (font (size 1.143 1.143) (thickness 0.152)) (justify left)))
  (pad "" np_thru_hole circle (at 0 0) (size 3 3) (drill 3) (layers "*.Cu" "*.Mask"))
  (pad 3 thru_hole oval (at 0 -4.92 -90) (size 2.7 1.7) (layers "*.Cu" "*.Paste" "*.Mask") (drill oval 0.5 1.5) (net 13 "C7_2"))
  (pad 2 thru_hole oval (at 0 3.38 -90) (size 2.7 1.7) (layers "*.Cu" "*.Paste" "*.Mask") (drill oval 0.5 1.5))
  (pad 1 thru_hole oval (at 0 6.48 -90) (size 2.7 1.7) (layers "*.Cu" "*.Paste" "*.Mask") (drill oval 0.5 1.5) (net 1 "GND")))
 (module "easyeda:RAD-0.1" (layer "F.Cu") (at 13.97 125.222)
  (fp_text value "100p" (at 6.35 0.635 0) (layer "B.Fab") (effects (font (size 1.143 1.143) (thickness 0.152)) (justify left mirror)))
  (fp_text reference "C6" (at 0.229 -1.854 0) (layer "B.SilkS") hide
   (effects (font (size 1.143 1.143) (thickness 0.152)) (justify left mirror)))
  (pad 1 thru_hole circle (at 1.27 0 0) (size 1.194 1.194) (layers "*.Cu" "*.Paste" "*.Mask") (drill 0.711) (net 11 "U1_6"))
  (pad 2 thru_hole circle (at -1.27 0 0) (size 1.194 1.194) (layers "*.Cu" "*.Paste" "*.Mask") (drill 0.711) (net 7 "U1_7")))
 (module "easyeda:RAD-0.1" (layer "F.Cu") (at 20.32 118.872 -90)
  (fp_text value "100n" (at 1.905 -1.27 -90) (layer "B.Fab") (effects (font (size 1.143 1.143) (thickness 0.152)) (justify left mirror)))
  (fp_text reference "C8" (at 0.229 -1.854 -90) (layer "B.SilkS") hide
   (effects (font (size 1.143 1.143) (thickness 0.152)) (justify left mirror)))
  (pad 1 thru_hole circle (at 1.27 0 -90) (size 1.194 1.194) (layers "*.Cu" "*.Paste" "*.Mask") (drill 0.711) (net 14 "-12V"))
  (pad 2 thru_hole circle (at -1.27 0 -90) (size 1.194 1.194) (layers "*.Cu" "*.Paste" "*.Mask") (drill 0.711) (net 1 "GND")))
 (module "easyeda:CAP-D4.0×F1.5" (layer "F.Cu") (at 7.62 91.567 -90)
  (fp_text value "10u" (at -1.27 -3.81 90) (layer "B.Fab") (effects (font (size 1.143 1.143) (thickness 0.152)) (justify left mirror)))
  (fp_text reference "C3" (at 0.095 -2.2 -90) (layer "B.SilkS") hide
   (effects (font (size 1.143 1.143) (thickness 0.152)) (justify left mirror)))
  (pad 2 thru_hole circle (at -0.751 0 180) (size 1 1) (layers "*.Cu" "*.Paste" "*.Mask") (drill 0.7) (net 14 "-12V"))
  (pad 1 thru_hole circle (at 0.751 0 180) (size 1 1) (layers "*.Cu" "*.Paste" "*.Mask") (drill 0.7) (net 1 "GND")))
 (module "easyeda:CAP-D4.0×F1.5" (layer "F.Cu") (at 7.62 97.917 -90)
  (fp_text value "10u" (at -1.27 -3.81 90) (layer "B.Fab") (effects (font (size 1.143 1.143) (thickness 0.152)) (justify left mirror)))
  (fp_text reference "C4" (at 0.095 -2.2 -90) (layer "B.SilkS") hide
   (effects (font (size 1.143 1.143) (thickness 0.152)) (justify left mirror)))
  (pad 2 thru_hole circle (at -0.751 0 180) (size 1 1) (layers "*.Cu" "*.Paste" "*.Mask") (drill 0.7) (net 1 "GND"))
  (pad 1 thru_hole circle (at 0.751 0 180) (size 1 1) (layers "*.Cu" "*.Paste" "*.Mask") (drill 0.7) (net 15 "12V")))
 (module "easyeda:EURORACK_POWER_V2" (layer "F.Cu") (at 14.351 95.123 -90)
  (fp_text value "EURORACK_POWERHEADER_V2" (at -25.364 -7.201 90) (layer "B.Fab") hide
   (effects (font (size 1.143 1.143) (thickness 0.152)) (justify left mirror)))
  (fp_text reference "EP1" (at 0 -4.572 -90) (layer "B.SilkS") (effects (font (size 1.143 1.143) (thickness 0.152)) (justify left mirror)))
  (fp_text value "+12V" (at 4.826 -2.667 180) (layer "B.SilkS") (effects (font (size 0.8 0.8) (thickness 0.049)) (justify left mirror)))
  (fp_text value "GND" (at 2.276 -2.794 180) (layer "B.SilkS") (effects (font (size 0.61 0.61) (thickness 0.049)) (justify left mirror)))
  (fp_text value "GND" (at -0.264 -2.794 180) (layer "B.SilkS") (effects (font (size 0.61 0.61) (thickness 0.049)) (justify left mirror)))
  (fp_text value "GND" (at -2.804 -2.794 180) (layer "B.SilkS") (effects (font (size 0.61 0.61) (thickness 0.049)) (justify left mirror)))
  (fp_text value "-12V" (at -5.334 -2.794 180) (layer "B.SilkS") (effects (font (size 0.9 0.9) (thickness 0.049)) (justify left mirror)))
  (pad 12 thru_hole custom (at 5.08 -1.27 -90) (size 1.408 1.408) (layers "*.Cu" "*.Paste" "*.Mask") (drill oval 1.016 1.021) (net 15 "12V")
   (primitives))
  (pad 12 thru_hole custom (at 5.08 1.27 -90) (size 0.01 0.01) (layers "*.Cu" "*.Paste" "*.Mask") (drill oval 1.016 1.021) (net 15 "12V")
   (primitives))
  (pad -12 thru_hole custom (at -5.08 -1.27 -90) (size 1.408 1.408) (layers "*.Cu" "*.Paste" "*.Mask") (drill oval 1.016 1.021)
   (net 14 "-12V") (primitives))
  (pad -12 thru_hole custom (at -5.08 1.27 -90) (size 1.408 1.408) (layers "*.Cu" "*.Paste" "*.Mask") (drill oval 1.016 1.021)
   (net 14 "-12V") (primitives))
  (pad "GND0" thru_hole custom (at 2.54 -1.27 -90) (size 1.408 1.408) (layers "*.Cu" "*.Paste" "*.Mask") (drill oval 1.016 1.021)
   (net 1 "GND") (primitives))
  (pad "GND1" thru_hole custom (at 2.54 1.27 180) (size 0.01 0.01) (layers "*.Cu" "*.Paste" "*.Mask") (drill oval 1.016 1.021) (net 1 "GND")
   (primitives))
  (pad "GND2" thru_hole custom (at 0 -1.27 -90) (size 1.408 1.408) (layers "*.Cu" "*.Paste" "*.Mask") (drill oval 1.016 1.021) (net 1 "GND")
   (primitives))
  (pad "GND3" thru_hole custom (at 0 1.27 -90) (size 1.408 1.408) (layers "*.Cu" "*.Paste" "*.Mask") (drill oval 1.016 1.021) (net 1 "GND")
   (primitives))
  (pad "GND4" thru_hole custom (at -2.54 -1.27 -90) (size 1.408 1.408) (layers "*.Cu" "*.Paste" "*.Mask") (drill oval 1.016 1.021)
   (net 1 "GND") (primitives))
  (pad "GND5" thru_hole custom (at -2.54 1.27 -90) (size 1.408 1.408) (layers "*.Cu" "*.Paste" "*.Mask") (drill oval 1.016 1.021)
   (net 1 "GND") (primitives)))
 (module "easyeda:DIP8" (layer "F.Cu") (at 13.97 118.872 180)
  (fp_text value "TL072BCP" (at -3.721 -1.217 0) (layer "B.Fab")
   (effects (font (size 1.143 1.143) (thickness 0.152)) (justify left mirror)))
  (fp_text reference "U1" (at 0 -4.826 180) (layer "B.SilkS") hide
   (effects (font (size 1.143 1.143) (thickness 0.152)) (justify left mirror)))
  (pad 1 thru_hole rect (at 3.81 3.81 180) (size 1.397 1.397) (layers "*.Cu" "*.Paste" "*.Mask") (drill 0.711) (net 5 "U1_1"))
  (pad 2 thru_hole circle (at 1.27 3.81 180) (size 1.397 1.397) (layers "*.Cu" "*.Paste" "*.Mask") (drill 0.711) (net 8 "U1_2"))
  (pad 3 thru_hole circle (at -1.27 3.81 180) (size 1.397 1.397) (layers "*.Cu" "*.Paste" "*.Mask") (drill 0.711) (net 1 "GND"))
  (pad 4 thru_hole circle (at -3.81 3.81 180) (size 1.397 1.397) (layers "*.Cu" "*.Paste" "*.Mask") (drill 0.711) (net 14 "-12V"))
  (pad 5 thru_hole circle (at -3.81 -3.81 180) (size 1.397 1.397) (layers "*.Cu" "*.Paste" "*.Mask") (drill 0.711) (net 1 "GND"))
  (pad 6 thru_hole circle (at -1.27 -3.81 180) (size 1.397 1.397) (layers "*.Cu" "*.Paste" "*.Mask") (drill 0.711) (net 11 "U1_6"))
  (pad 7 thru_hole circle (at 1.27 -3.81 180) (size 1.397 1.397) (layers "*.Cu" "*.Paste" "*.Mask") (drill 0.711) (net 7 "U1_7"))
  (pad 8 thru_hole circle (at 3.81 -3.81 180) (size 1.397 1.397) (layers "*.Cu" "*.Paste" "*.Mask") (drill 0.711) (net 15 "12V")))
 (via (at 20.21 149.429) (size 0.75) (drill 0.58) (layers "F.Cu" "B.Cu") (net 1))
 (via (at 15.154 104.756) (size 0.7) (drill 0.5) (layers "F.Cu" "B.Cu") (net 3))
 (via (at 13.79 120.434) (size 0.7) (drill 0.5) (layers "F.Cu" "B.Cu") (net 5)))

